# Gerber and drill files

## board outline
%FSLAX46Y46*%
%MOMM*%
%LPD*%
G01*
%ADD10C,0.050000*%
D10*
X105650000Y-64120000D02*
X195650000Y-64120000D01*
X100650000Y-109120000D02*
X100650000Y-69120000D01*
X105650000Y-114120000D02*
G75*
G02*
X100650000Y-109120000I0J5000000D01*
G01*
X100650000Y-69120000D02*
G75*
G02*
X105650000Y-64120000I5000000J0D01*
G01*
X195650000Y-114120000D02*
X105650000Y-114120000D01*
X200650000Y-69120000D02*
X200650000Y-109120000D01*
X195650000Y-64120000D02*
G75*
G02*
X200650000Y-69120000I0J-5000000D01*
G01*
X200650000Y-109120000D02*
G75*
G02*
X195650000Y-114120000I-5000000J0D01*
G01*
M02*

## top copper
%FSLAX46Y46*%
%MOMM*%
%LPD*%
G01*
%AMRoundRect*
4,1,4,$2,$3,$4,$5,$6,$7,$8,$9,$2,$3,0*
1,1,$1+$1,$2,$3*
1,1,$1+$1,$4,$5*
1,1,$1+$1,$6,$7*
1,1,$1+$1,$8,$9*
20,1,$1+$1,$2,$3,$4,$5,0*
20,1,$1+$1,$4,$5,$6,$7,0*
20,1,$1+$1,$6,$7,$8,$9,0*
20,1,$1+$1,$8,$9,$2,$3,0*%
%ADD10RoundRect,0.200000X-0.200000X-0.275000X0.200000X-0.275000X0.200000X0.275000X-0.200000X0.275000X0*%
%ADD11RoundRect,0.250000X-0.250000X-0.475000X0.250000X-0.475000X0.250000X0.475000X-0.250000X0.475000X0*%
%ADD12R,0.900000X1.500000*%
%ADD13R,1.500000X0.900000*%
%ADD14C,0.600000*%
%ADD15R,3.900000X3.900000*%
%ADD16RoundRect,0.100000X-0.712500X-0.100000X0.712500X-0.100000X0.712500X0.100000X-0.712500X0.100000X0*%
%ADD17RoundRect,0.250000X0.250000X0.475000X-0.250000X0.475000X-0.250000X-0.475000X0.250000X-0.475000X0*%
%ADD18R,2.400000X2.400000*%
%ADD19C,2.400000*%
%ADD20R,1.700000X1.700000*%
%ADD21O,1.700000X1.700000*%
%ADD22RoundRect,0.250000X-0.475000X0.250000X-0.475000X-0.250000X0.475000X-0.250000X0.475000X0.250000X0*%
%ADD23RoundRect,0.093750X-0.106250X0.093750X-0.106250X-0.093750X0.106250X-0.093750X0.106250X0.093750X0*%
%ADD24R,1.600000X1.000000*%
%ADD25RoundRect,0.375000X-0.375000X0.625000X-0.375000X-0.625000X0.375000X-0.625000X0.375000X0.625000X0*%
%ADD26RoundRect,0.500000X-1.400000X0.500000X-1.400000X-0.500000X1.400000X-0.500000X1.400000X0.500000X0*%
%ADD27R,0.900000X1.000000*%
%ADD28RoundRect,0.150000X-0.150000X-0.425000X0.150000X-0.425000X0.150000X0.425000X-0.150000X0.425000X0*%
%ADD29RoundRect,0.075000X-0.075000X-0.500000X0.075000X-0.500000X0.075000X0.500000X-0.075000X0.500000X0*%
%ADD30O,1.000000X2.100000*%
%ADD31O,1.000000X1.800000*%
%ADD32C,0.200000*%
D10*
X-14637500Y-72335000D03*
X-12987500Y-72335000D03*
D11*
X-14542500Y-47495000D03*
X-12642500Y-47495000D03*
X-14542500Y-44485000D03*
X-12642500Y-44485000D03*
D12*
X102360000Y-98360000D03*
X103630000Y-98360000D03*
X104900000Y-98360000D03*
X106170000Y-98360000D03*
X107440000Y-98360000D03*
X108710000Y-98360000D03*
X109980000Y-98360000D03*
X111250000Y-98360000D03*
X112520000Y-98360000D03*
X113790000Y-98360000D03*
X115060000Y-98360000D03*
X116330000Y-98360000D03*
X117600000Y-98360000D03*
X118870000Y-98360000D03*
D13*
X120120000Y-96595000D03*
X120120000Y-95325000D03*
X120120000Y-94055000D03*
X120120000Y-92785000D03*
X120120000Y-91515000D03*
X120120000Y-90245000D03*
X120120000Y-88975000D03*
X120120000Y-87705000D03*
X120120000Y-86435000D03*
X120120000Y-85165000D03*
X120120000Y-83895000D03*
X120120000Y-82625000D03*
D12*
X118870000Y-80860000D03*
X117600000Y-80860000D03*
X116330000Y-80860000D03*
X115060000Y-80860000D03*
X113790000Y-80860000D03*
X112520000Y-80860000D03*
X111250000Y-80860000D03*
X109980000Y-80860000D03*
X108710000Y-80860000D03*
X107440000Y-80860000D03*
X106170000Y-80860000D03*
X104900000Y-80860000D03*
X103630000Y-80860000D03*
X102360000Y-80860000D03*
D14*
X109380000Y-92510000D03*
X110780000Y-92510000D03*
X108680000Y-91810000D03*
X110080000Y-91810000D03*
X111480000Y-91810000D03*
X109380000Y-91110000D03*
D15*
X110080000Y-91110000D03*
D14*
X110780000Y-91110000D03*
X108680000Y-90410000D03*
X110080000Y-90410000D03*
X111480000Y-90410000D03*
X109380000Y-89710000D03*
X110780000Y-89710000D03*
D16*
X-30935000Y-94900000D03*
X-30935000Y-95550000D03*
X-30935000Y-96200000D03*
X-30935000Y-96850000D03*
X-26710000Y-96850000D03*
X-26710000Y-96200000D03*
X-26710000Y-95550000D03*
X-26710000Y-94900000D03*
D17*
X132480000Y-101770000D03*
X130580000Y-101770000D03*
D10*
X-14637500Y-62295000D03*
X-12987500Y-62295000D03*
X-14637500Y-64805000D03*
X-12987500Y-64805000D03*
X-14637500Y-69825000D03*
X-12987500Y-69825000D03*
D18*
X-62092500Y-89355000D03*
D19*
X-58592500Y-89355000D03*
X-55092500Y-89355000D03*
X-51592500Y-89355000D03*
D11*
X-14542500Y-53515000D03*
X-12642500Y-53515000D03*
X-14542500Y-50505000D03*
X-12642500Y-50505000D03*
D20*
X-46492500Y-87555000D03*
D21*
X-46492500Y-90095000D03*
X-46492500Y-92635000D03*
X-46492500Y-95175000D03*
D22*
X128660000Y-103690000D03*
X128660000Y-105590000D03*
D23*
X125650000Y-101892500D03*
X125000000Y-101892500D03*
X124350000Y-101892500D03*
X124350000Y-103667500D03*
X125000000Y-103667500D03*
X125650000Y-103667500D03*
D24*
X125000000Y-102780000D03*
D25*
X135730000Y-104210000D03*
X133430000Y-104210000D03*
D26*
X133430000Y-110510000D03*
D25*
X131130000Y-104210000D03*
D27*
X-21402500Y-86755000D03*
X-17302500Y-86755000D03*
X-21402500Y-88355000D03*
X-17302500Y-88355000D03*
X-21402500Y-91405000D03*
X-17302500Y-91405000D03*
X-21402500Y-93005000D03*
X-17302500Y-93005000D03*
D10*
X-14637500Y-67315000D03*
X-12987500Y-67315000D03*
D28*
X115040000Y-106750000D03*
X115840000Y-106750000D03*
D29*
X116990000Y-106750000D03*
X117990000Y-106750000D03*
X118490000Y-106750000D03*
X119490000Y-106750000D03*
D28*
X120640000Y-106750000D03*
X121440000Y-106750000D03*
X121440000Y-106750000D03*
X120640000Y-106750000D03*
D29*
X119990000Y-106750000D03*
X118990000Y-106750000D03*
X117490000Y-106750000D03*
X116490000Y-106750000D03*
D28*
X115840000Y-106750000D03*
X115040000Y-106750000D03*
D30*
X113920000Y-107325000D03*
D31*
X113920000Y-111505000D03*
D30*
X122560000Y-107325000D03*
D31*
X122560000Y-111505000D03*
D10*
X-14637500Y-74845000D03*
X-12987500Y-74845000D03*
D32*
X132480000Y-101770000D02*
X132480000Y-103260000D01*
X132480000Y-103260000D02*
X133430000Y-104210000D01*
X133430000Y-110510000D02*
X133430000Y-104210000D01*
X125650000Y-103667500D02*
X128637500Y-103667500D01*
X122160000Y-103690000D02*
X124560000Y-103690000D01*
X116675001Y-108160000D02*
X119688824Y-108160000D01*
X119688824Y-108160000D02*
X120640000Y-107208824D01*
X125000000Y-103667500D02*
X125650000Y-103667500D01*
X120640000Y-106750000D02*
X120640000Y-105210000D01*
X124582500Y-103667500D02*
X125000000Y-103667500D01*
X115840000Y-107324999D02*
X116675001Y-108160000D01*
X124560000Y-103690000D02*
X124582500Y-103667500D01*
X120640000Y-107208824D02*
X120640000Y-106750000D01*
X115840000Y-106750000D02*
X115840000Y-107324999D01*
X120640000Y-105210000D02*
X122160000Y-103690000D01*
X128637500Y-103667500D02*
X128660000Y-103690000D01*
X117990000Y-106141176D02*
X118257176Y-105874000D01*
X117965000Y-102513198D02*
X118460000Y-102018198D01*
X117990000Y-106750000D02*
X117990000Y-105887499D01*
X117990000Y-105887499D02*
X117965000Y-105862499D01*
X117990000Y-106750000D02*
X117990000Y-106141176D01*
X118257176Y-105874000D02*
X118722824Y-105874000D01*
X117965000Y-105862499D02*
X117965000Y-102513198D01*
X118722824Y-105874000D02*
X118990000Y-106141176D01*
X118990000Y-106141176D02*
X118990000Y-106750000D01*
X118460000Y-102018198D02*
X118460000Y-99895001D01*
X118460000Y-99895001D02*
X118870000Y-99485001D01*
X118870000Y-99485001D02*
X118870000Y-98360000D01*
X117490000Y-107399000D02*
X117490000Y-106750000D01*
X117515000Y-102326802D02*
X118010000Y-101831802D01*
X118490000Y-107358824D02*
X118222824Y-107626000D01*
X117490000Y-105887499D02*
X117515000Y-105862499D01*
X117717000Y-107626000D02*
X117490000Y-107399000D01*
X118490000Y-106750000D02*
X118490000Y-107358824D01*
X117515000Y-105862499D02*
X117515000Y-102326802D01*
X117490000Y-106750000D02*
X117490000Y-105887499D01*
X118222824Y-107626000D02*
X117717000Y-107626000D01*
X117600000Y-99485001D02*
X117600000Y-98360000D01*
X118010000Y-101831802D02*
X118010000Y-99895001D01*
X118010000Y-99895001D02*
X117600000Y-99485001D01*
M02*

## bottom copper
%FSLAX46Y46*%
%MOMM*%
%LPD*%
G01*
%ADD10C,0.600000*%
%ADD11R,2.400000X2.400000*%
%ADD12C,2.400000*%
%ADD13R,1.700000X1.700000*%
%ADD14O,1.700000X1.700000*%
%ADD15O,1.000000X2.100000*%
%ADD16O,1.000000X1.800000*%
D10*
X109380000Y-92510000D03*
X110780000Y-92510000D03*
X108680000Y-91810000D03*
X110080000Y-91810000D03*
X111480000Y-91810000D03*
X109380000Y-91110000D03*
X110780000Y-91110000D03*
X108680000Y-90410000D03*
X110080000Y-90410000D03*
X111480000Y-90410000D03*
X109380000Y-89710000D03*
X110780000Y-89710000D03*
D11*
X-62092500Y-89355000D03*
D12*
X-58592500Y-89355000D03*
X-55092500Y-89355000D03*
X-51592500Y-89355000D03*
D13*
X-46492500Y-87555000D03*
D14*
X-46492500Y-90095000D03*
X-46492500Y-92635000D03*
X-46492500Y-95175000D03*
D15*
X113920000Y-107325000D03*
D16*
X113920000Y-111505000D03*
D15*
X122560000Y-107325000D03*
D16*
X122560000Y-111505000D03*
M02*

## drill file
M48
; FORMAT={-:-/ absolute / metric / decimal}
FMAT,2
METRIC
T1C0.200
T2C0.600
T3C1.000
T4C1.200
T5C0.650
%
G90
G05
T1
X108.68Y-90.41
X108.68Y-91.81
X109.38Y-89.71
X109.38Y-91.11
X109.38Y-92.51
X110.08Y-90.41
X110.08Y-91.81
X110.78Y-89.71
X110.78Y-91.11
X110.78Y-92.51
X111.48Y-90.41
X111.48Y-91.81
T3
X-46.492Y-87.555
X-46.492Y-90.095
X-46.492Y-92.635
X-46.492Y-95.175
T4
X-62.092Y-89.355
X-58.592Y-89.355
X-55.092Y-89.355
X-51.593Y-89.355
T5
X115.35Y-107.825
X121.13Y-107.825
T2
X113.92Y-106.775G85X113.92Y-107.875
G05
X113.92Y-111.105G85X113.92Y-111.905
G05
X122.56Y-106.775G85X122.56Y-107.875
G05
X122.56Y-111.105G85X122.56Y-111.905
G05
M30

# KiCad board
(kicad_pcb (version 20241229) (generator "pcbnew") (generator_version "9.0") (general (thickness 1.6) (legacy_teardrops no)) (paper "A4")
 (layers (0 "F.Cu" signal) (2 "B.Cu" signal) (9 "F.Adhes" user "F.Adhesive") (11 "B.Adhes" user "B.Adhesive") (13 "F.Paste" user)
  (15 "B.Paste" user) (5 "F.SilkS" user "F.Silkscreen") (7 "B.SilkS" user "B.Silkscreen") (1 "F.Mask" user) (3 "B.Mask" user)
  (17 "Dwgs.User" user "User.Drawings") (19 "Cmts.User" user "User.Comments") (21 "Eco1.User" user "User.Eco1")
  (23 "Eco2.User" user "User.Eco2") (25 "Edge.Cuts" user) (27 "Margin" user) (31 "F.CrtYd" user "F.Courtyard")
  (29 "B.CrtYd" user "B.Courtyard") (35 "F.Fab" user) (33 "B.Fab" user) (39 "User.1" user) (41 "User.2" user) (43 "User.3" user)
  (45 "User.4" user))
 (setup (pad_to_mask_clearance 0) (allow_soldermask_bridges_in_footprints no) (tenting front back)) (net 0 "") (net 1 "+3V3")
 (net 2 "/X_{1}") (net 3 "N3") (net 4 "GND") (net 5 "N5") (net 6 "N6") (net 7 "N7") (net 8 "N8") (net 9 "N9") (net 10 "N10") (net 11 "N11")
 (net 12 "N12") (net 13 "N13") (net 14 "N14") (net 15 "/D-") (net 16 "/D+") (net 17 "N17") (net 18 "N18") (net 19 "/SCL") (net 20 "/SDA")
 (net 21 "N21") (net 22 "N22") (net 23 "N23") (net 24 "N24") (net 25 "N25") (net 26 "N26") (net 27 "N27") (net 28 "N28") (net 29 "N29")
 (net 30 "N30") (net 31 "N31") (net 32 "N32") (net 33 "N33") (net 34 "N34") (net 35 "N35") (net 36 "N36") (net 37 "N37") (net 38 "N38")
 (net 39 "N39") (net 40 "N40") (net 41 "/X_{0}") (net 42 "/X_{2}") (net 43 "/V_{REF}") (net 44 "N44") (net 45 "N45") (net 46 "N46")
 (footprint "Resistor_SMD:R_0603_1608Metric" (layer "F.Cu") (at -13.8125 72.335)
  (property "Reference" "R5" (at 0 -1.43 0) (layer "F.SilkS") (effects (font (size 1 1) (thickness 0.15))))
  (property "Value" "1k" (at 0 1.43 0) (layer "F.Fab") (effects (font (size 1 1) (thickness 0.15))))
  (pad "1" smd roundrect (at -0.825 0) (size 0.8 0.95) (layers "F.Cu" "F.Mask" "F.Paste") (roundrect_rratio 0.25) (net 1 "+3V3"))
  (pad "2" smd roundrect (at 0.825 0) (size 0.8 0.95) (layers "F.Cu" "F.Mask" "F.Paste") (roundrect_rratio 0.25) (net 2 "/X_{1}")))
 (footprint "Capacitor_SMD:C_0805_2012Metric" (layer "F.Cu") (at -13.5925 47.495)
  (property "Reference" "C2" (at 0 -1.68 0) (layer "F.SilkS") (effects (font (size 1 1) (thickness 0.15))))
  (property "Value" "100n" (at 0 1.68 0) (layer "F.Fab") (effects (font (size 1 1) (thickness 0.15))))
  (pad "1" smd roundrect (at -0.95 0) (size 1 1.45) (layers "F.Cu" "F.Mask" "F.Paste") (roundrect_rratio 0.25) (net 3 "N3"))
  (pad "2" smd roundrect (at 0.95 0) (size 1 1.45) (layers "F.Cu" "F.Mask" "F.Paste") (roundrect_rratio 0.25) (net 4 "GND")))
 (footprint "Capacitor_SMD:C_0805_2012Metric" (layer "F.Cu") (at -13.5925 44.485)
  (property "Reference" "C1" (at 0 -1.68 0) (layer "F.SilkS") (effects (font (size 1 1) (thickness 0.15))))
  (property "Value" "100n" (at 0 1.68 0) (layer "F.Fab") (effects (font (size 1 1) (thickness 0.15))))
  (pad "1" smd roundrect (at -0.95 0) (size 1 1.45) (layers "F.Cu" "F.Mask" "F.Paste") (roundrect_rratio 0.25) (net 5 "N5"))
  (pad "2" smd roundrect (at 0.95 0) (size 1 1.45) (layers "F.Cu" "F.Mask" "F.Paste") (roundrect_rratio 0.25) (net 4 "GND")))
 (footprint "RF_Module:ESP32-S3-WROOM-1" (layer "F.Cu") (at 107.62 89.61 90)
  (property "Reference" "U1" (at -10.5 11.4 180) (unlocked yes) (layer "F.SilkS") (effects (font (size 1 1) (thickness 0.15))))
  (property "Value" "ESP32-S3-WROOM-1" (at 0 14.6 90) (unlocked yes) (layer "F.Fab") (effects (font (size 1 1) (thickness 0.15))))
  (pad "" smd rect (at -2.9 1.06 90) (size 0.9 0.9) (layers "F.Paste"))
  (pad "" smd rect (at -2.9 2.46) (size 0.9 0.9) (layers "F.Paste"))
  (pad "" smd rect (at -2.9 3.86 90) (size 0.9 0.9) (layers "F.Paste"))
  (pad "" smd rect (at -1.5 1.06) (size 0.9 0.9) (layers "F.Paste"))
  (pad "" smd rect (at -1.5 2.46) (size 0.9 0.9) (layers "F.Paste"))
  (pad "" smd rect (at -1.5 3.86) (size 0.9 0.9) (layers "F.Paste"))
  (pad "" smd rect (at -0.1 1.06) (size 0.9 0.9) (layers "F.Paste"))
  (pad "" smd rect (at -0.1 2.46) (size 0.9 0.9) (layers "F.Paste"))
  (pad "" smd rect (at -0.1 3.86) (size 0.9 0.9) (layers "F.Paste"))
  (pad "1" smd rect (at -8.75 -5.26 90) (size 1.5 0.9) (layers "F.Cu" "F.Mask" "F.Paste") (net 4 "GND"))
  (pad "2" smd rect (at -8.75 -3.99 90) (size 1.5 0.9) (layers "F.Cu" "F.Mask" "F.Paste") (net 1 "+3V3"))
  (pad "3" smd rect (at -8.75 -2.72 90) (size 1.5 0.9) (layers "F.Cu" "F.Mask" "F.Paste") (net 5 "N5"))
  (pad "4" smd rect (at -8.75 -1.45 90) (size 1.5 0.9) (layers "F.Cu" "F.Mask" "F.Paste") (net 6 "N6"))
  (pad "5" smd rect (at -8.75 -0.18 90) (size 1.5 0.9) (layers "F.Cu" "F.Mask" "F.Paste") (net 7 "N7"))
  (pad "6" smd rect (at -8.75 1.09 90) (size 1.5 0.9) (layers "F.Cu" "F.Mask" "F.Paste") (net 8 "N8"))
  (pad "7" smd rect (at -8.75 2.36 90) (size 1.5 0.9) (layers "F.Cu" "F.Mask" "F.Paste") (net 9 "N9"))
  (pad "8" smd rect (at -8.75 3.63 90) (size 1.5 0.9) (layers "F.Cu" "F.Mask" "F.Paste") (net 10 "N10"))
  (pad "9" smd rect (at -8.75 4.9 90) (size 1.5 0.9) (layers "F.Cu" "F.Mask" "F.Paste") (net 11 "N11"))
  (pad "10" smd rect (at -8.75 6.17 90) (size 1.5 0.9) (layers "F.Cu" "F.Mask" "F.Paste") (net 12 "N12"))
  (pad "11" smd rect (at -8.75 7.44 90) (size 1.5 0.9) (layers "F.Cu" "F.Mask" "F.Paste") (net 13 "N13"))
  (pad "12" smd rect (at -8.75 8.71 90) (size 1.5 0.9) (layers "F.Cu" "F.Mask" "F.Paste") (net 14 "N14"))
  (pad "13" smd rect (at -8.75 9.98 90) (size 1.5 0.9) (layers "F.Cu" "F.Mask" "F.Paste") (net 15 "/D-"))
  (pad "14" smd rect (at -8.75 11.25 270) (size 1.5 0.9) (layers "F.Cu" "F.Mask" "F.Paste") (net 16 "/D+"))
  (pad "15" smd rect (at -6.985 12.5) (size 1.5 0.9) (layers "F.Cu" "F.Mask" "F.Paste") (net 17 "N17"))
  (pad "16" smd rect (at -5.715 12.5) (size 1.5 0.9) (layers "F.Cu" "F.Mask" "F.Paste") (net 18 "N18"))
  (pad "17" smd rect (at -4.445 12.5) (size 1.5 0.9) (layers "F.Cu" "F.Mask" "F.Paste") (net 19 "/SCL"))
  (pad "18" smd rect (at -3.175 12.5) (size 1.5 0.9) (layers "F.Cu" "F.Mask" "F.Paste") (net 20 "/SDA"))
  (pad "19" smd rect (at -1.905 12.5) (size 1.5 0.9) (layers "F.Cu" "F.Mask" "F.Paste") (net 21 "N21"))
  (pad "20" smd rect (at -0.635 12.5) (size 1.5 0.9) (layers "F.Cu" "F.Mask" "F.Paste") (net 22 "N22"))
  (pad "21" smd rect (at 0.635 12.5) (size 1.5 0.9) (layers "F.Cu" "F.Mask" "F.Paste") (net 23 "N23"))
  (pad "22" smd rect (at 1.905 12.5) (size 1.5 0.9) (layers "F.Cu" "F.Mask" "F.Paste") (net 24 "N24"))
  (pad "23" smd rect (at 3.175 12.5) (size 1.5 0.9) (layers "F.Cu" "F.Mask" "F.Paste") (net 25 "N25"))
  (pad "24" smd rect (at 4.445 12.5) (size 1.5 0.9) (layers "F.Cu" "F.Mask" "F.Paste") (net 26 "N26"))
  (pad "25" smd rect (at 5.715 12.5) (size 1.5 0.9) (layers "F.Cu" "F.Mask" "F.Paste") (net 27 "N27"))
  (pad "26" smd rect (at 6.985 12.5) (size 1.5 0.9) (layers "F.Cu" "F.Mask" "F.Paste") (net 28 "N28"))
  (pad "27" smd rect (at 8.75 11.25 90) (size 1.5 0.9) (layers "F.Cu" "F.Mask" "F.Paste") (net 3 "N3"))
  (pad "28" smd rect (at 8.75 9.98 90) (size 1.5 0.9) (layers "F.Cu" "F.Mask" "F.Paste") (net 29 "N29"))
  (pad "29" smd rect (at 8.75 8.71 90) (size 1.5 0.9) (layers "F.Cu" "F.Mask" "F.Paste") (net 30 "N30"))
  (pad "30" smd rect (at 8.75 7.44 90) (size 1.5 0.9) (layers "F.Cu" "F.Mask" "F.Paste") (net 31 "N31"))
  (pad "31" smd rect (at 8.75 6.17 90) (size 1.5 0.9) (layers "F.Cu" "F.Mask" "F.Paste") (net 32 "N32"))
  (pad "32" smd rect (at 8.75 4.9 90) (size 1.5 0.9) (layers "F.Cu" "F.Mask" "F.Paste") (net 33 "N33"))
  (pad "33" smd rect (at 8.75 3.63 90) (size 1.5 0.9) (layers "F.Cu" "F.Mask" "F.Paste") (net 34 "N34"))
  (pad "34" smd rect (at 8.75 2.36 90) (size 1.5 0.9) (layers "F.Cu" "F.Mask" "F.Paste") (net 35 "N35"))
  (pad "35" smd rect (at 8.75 1.09 90) (size 1.5 0.9) (layers "F.Cu" "F.Mask" "F.Paste") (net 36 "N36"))
  (pad "36" smd rect (at 8.75 -0.18 90) (size 1.5 0.9) (layers "F.Cu" "F.Mask" "F.Paste") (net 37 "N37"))
  (pad "37" smd rect (at 8.75 -1.45 90) (size 1.5 0.9) (layers "F.Cu" "F.Mask" "F.Paste") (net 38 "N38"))
  (pad "38" smd rect (at 8.75 -2.72 90) (size 1.5 0.9) (layers "F.Cu" "F.Mask" "F.Paste") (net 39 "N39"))
  (pad "39" smd rect (at 8.75 -3.99 90) (size 1.5 0.9) (layers "F.Cu" "F.Mask" "F.Paste") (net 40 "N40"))
  (pad "40" smd rect (at 8.75 -5.26 90) (size 1.5 0.9) (layers "F.Cu" "F.Mask" "F.Paste") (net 4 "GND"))
  (pad "41" thru_hole circle (at -2.9 1.76 180) (size 0.6 0.6) (drill 0.2) (layers "*.Cu" "F.Mask") (remove_unused_layers no) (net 4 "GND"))
  (pad "41" thru_hole circle (at -2.9 3.16 90) (size 0.6 0.6) (drill 0.2) (layers "*.Cu" "F.Mask") (remove_unused_layers no) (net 4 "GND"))
  (pad "41" thru_hole circle (at -2.2 1.06 90) (size 0.6 0.6) (drill 0.2) (layers "*.Cu" "F.Mask") (remove_unused_layers no) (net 4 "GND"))
  (pad "41" thru_hole circle (at -2.2 2.46 90) (size 0.6 0.6) (drill 0.2) (layers "*.Cu" "F.Mask") (remove_unused_layers no) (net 4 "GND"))
  (pad "41" thru_hole circle (at -2.2 3.86 90) (size 0.6 0.6) (drill 0.2) (layers "*.Cu" "F.Mask") (remove_unused_layers no) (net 4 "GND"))
  (pad "41" thru_hole circle (at -1.5 1.76 90) (size 0.6 0.6) (drill 0.2) (layers "*.Cu" "F.Mask") (remove_unused_layers no) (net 4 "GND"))
  (pad "41" smd rect (at -1.5 2.46) (size 3.9 3.9) (layers "F.Cu" "F.Mask") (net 4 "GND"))
  (pad "41" thru_hole circle (at -1.5 3.16 90) (size 0.6 0.6) (drill 0.2) (layers "*.Cu" "F.Mask") (remove_unused_layers no) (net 4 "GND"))
  (pad "41" thru_hole circle (at -0.8 1.06 90) (size 0.6 0.6) (drill 0.2) (layers "*.Cu" "F.Mask") (remove_unused_layers no) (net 4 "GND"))
  (pad "41" thru_hole circle (at -0.8 2.46 90) (size 0.6 0.6) (drill 0.2) (layers "*.Cu" "F.Mask") (remove_unused_layers no) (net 4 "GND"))
  (pad "41" thru_hole circle (at -0.8 3.86 90) (size 0.6 0.6) (drill 0.2) (layers "*.Cu" "F.Mask") (remove_unused_layers no) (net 4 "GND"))
  (pad "41" thru_hole circle (at -0.1 1.76 90) (size 0.6 0.6) (drill 0.2) (layers "*.Cu" "F.Mask") (remove_unused_layers no) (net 4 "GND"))
  (pad "41" thru_hole circle (at -0.1 3.16 90) (size 0.6 0.6) (drill 0.2) (layers "*.Cu" "F.Mask") (remove_unused_layers no) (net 4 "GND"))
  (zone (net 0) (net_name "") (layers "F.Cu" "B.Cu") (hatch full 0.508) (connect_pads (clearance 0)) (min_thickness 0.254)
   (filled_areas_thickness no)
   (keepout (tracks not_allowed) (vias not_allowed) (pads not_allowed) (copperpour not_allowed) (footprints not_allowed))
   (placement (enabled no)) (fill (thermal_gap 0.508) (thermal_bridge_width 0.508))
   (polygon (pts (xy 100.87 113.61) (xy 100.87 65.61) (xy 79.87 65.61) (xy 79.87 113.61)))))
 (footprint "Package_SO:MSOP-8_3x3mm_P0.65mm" (layer "F.Cu") (at -28.8225 95.875)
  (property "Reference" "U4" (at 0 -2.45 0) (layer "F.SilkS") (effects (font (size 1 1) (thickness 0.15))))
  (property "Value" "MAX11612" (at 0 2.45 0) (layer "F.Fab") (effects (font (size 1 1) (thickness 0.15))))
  (pad "1" smd roundrect (at -2.1125 -0.975) (size 1.625 0.4) (layers "F.Cu" "F.Mask" "F.Paste") (roundrect_rratio 0.25) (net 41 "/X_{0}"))
  (pad "2" smd roundrect (at -2.1125 -0.325) (size 1.625 0.4) (layers "F.Cu" "F.Mask" "F.Paste") (roundrect_rratio 0.25) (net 2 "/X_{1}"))
  (pad "3" smd roundrect (at -2.1125 0.325) (size 1.625 0.4) (layers "F.Cu" "F.Mask" "F.Paste") (roundrect_rratio 0.25) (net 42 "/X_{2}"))
  (pad "4" smd roundrect (at -2.1125 0.975) (size 1.625 0.4) (layers "F.Cu" "F.Mask" "F.Paste") (roundrect_rratio 0.25) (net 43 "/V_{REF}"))
  (pad "5" smd roundrect (at 2.1125 0.975) (size 1.625 0.4) (layers "F.Cu" "F.Mask" "F.Paste") (roundrect_rratio 0.25) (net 19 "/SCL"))
  (pad "6" smd roundrect (at 2.1125 0.325) (size 1.625 0.4) (layers "F.Cu" "F.Mask" "F.Paste") (roundrect_rratio 0.25) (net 20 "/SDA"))
  (pad "7" smd roundrect (at 2.1125 -0.325) (size 1.625 0.4) (layers "F.Cu" "F.Mask" "F.Paste") (roundrect_rratio 0.25) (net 4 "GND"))
  (pad "8" smd roundrect (at 2.1125 -0.975) (size 1.625 0.4) (layers "F.Cu" "F.Mask" "F.Paste") (roundrect_rratio 0.25) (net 1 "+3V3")))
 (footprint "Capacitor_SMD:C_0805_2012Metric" (layer "F.Cu") (at 131.53 101.77 180)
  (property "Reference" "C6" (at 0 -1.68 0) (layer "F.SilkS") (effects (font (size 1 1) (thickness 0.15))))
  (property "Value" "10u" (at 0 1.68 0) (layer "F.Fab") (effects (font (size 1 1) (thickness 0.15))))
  (pad "1" smd roundrect (at -0.95 0 180) (size 1 1.45) (layers "F.Cu" "F.Mask" "F.Paste") (roundrect_rratio 0.25) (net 1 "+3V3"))
  (pad "2" smd roundrect (at 0.95 0 180) (size 1 1.45) (layers "F.Cu" "F.Mask" "F.Paste") (roundrect_rratio 0.25) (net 4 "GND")))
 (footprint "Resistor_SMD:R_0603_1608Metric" (layer "F.Cu") (at -13.8125 62.295)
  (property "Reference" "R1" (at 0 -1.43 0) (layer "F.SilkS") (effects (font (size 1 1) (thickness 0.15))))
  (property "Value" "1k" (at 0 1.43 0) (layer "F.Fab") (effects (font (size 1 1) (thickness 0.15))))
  (pad "1" smd roundrect (at -0.825 0) (size 0.8 0.95) (layers "F.Cu" "F.Mask" "F.Paste") (roundrect_rratio 0.25) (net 1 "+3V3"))
  (pad "2" smd roundrect (at 0.825 0) (size 0.8 0.95) (layers "F.Cu" "F.Mask" "F.Paste") (roundrect_rratio 0.25) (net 5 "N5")))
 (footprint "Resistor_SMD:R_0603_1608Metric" (layer "F.Cu") (at -13.8125 64.805)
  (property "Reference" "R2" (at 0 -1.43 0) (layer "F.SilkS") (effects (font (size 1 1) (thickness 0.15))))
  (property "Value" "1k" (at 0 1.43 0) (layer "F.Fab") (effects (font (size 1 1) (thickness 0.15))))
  (pad "1" smd roundrect (at -0.825 0) (size 0.8 0.95) (layers "F.Cu" "F.Mask" "F.Paste") (roundrect_rratio 0.25) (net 1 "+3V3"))
  (pad "2" smd roundrect (at 0.825 0) (size 0.8 0.95) (layers "F.Cu" "F.Mask" "F.Paste") (roundrect_rratio 0.25) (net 3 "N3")))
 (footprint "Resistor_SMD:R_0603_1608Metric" (layer "F.Cu") (at -13.8125 69.825)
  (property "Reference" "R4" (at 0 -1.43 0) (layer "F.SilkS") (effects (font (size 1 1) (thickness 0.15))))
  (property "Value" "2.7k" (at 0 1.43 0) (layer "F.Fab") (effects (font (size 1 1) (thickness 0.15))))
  (pad "1" smd roundrect (at -0.825 0) (size 0.8 0.95) (layers "F.Cu" "F.Mask" "F.Paste") (roundrect_rratio 0.25) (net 1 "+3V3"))
  (pad "2" smd roundrect (at 0.825 0) (size 0.8 0.95) (layers "F.Cu" "F.Mask" "F.Paste") (roundrect_rratio 0.25) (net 20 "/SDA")))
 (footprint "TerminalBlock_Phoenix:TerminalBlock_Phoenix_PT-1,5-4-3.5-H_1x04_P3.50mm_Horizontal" (layer "F.Cu") (at -62.0925 89.355)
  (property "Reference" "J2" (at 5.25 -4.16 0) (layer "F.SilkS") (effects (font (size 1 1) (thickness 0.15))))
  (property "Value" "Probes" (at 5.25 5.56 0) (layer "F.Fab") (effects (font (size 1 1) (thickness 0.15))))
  (pad "1" thru_hole rect (at 0 0) (size 2.4 2.4) (drill 1.2) (layers "*.Cu" "*.Mask") (remove_unused_layers no) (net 41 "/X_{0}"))
  (pad "2" thru_hole circle (at 3.5 0) (size 2.4 2.4) (drill 1.2) (layers "*.Cu" "*.Mask") (remove_unused_layers no) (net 2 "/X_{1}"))
  (pad "3" thru_hole circle (at 7 0) (size 2.4 2.4) (drill 1.2) (layers "*.Cu" "*.Mask") (remove_unused_layers no) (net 42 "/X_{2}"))
  (pad "4" thru_hole circle (at 10.5 0) (size 2.4 2.4) (drill 1.2) (layers "*.Cu" "*.Mask") (remove_unused_layers no) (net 43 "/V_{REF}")))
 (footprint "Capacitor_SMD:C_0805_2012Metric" (layer "F.Cu") (at -13.5925 53.515)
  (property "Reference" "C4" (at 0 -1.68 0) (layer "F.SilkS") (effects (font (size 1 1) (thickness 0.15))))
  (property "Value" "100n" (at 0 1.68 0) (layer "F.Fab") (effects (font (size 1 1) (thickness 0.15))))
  (pad "1" smd roundrect (at -0.95 0) (size 1 1.45) (layers "F.Cu" "F.Mask" "F.Paste") (roundrect_rratio 0.25) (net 1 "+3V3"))
  (pad "2" smd roundrect (at 0.95 0) (size 1 1.45) (layers "F.Cu" "F.Mask" "F.Paste") (roundrect_rratio 0.25) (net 4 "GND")))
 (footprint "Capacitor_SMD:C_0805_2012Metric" (layer "F.Cu") (at -13.5925 50.505)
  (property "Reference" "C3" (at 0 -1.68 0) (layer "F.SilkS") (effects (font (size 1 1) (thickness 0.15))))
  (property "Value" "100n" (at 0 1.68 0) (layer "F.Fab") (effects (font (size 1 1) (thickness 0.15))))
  (pad "1" smd roundrect (at -0.95 0) (size 1 1.45) (layers "F.Cu" "F.Mask" "F.Paste") (roundrect_rratio 0.25) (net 1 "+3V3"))
  (pad "2" smd roundrect (at 0.95 0) (size 1 1.45) (layers "F.Cu" "F.Mask" "F.Paste") (roundrect_rratio 0.25) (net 4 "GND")))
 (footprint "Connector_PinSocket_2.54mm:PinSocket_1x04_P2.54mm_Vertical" (layer "F.Cu") (at -46.4925 87.555)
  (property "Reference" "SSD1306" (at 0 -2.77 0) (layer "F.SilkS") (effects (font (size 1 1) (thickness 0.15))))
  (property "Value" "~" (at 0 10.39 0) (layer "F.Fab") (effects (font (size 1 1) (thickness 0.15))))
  (pad "1" thru_hole rect (at 0 0) (size 1.7 1.7) (drill 1) (layers "*.Cu" "*.Mask") (remove_unused_layers no) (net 4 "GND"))
  (pad "2" thru_hole oval (at 0 2.54) (size 1.7 1.7) (drill 1) (layers "*.Cu" "*.Mask") (remove_unused_layers no) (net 1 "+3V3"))
  (pad "3" thru_hole oval (at 0 5.08) (size 1.7 1.7) (drill 1) (layers "*.Cu" "*.Mask") (remove_unused_layers no) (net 19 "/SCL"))
  (pad "4" thru_hole oval (at 0 7.62) (size 1.7 1.7) (drill 1) (layers "*.Cu" "*.Mask") (remove_unused_layers no) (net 20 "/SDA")))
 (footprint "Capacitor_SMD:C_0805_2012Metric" (layer "F.Cu") (at 128.66 104.64 -90)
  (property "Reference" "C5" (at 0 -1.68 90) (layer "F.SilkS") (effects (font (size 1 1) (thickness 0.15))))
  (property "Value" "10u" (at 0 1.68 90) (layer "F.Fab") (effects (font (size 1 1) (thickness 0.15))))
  (pad "1" smd roundrect (at -0.95 0 270) (size 1 1.45) (layers "F.Cu" "F.Mask" "F.Paste") (roundrect_rratio 0.25) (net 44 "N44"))
  (pad "2" smd roundrect (at 0.95 0 270) (size 1 1.45) (layers "F.Cu" "F.Mask" "F.Paste") (roundrect_rratio 0.25) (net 4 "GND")))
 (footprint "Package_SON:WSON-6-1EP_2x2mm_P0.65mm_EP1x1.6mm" (layer "F.Cu") (at 125 102.78 -90)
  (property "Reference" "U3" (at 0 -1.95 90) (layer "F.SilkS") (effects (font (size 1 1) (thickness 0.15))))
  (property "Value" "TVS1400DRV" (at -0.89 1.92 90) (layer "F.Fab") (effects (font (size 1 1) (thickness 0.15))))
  (pad "" smd roundrect (at 0 -0.4 270) (size 0.81 0.64) (layers "F.Paste") (roundrect_rratio 0.25))
  (pad "" smd roundrect (at 0 0.4 270) (size 0.81 0.64) (layers "F.Paste") (roundrect_rratio 0.25))
  (pad "1" smd roundrect (at -0.8875 -0.65 270) (size 0.375 0.4) (layers "F.Cu" "F.Mask" "F.Paste") (roundrect_rratio 0.25) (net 4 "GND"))
  (pad "2" smd roundrect (at -0.8875 0 270) (size 0.375 0.4) (layers "F.Cu" "F.Mask" "F.Paste") (roundrect_rratio 0.25) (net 4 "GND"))
  (pad "3" smd roundrect (at -0.8875 0.65 270) (size 0.375 0.4) (layers "F.Cu" "F.Mask" "F.Paste") (roundrect_rratio 0.25) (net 4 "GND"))
  (pad "4" smd roundrect (at 0.8875 0.65 270) (size 0.375 0.4) (layers "F.Cu" "F.Mask" "F.Paste") (roundrect_rratio 0.25) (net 44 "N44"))
  (pad "5" smd roundrect (at 0.8875 0 270) (size 0.375 0.4) (layers "F.Cu" "F.Mask" "F.Paste") (roundrect_rratio 0.25) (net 44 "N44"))
  (pad "6" smd roundrect (at 0.8875 -0.65 270) (size 0.375 0.4) (layers "F.Cu" "F.Mask" "F.Paste") (roundrect_rratio 0.25) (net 44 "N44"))
  (pad "7" smd rect (at 0 0 270) (size 1 1.6) (layers "F.Cu" "F.Mask") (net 4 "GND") (zone_connect 2)))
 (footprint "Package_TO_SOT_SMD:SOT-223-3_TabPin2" (layer "F.Cu") (at 133.43 107.36 -90)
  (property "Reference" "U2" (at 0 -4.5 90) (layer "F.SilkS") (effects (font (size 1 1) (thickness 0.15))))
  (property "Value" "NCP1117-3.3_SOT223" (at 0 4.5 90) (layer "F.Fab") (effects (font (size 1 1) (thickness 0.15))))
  (pad "1" smd roundrect (at -3.15 -2.3 270) (size 2 1.5) (layers "F.Cu" "F.Mask" "F.Paste") (roundrect_rratio 0.25) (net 4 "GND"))
  (pad "2" smd roundrect (at -3.15 0 270) (size 2 1.5) (layers "F.Cu" "F.Mask" "F.Paste") (roundrect_rratio 0.25) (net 1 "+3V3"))
  (pad "2" smd roundrect (at 3.15 0 270) (size 2 3.8) (layers "F.Cu" "F.Mask" "F.Paste") (roundrect_rratio 0.25) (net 1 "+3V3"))
  (pad "3" smd roundrect (at -3.15 2.3 270) (size 2 1.5) (layers "F.Cu" "F.Mask" "F.Paste") (roundrect_rratio 0.25) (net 44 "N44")))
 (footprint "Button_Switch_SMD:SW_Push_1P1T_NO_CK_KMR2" (layer "F.Cu") (at -19.3525 87.555)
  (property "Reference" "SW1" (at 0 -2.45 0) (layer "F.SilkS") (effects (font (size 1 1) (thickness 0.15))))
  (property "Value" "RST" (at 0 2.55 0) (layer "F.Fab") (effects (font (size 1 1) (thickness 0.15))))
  (pad "1" smd rect (at -2.05 -0.8) (size 0.9 1) (layers "F.Cu" "F.Mask" "F.Paste") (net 4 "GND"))
  (pad "1" smd rect (at 2.05 -0.8) (size 0.9 1) (layers "F.Cu" "F.Mask" "F.Paste") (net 4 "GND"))
  (pad "2" smd rect (at -2.05 0.8) (size 0.9 1) (layers "F.Cu" "F.Mask" "F.Paste") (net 5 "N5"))
  (pad "2" smd rect (at 2.05 0.8) (size 0.9 1) (layers "F.Cu" "F.Mask" "F.Paste") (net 5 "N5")))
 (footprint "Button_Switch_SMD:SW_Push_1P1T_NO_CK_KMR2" (layer "F.Cu") (at -19.3525 92.205)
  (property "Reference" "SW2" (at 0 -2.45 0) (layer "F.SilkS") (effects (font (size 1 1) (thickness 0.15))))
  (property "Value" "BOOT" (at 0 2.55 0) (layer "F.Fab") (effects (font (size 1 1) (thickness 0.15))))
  (pad "1" smd rect (at -2.05 -0.8) (size 0.9 1) (layers "F.Cu" "F.Mask" "F.Paste") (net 4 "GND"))
  (pad "1" smd rect (at 2.05 -0.8) (size 0.9 1) (layers "F.Cu" "F.Mask" "F.Paste") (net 4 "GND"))
  (pad "2" smd rect (at -2.05 0.8) (size 0.9 1) (layers "F.Cu" "F.Mask" "F.Paste") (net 3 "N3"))
  (pad "2" smd rect (at 2.05 0.8) (size 0.9 1) (layers "F.Cu" "F.Mask" "F.Paste") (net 3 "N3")))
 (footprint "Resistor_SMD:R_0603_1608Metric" (layer "F.Cu") (at -13.8125 67.315)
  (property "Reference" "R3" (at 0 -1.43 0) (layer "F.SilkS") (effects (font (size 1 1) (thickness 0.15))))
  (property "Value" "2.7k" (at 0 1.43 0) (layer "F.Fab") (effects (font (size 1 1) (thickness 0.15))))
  (pad "1" smd roundrect (at -0.825 0) (size 0.8 0.95) (layers "F.Cu" "F.Mask" "F.Paste") (roundrect_rratio 0.25) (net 1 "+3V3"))
  (pad "2" smd roundrect (at 0.825 0) (size 0.8 0.95) (layers "F.Cu" "F.Mask" "F.Paste") (roundrect_rratio 0.25) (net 19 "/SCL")))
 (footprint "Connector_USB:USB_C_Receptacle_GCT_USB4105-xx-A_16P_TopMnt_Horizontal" (layer "F.Cu") (at 118.24 110.43)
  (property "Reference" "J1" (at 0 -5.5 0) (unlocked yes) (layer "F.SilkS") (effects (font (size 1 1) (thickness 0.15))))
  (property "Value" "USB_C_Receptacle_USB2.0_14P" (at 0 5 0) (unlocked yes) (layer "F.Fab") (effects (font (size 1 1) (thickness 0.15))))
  (pad "" np_thru_hole circle (at -2.89 -2.605) (size 0.65 0.65) (drill 0.65) (layers "*.Cu" "*.Mask"))
  (pad "" np_thru_hole circle (at 2.89 -2.605) (size 0.65 0.65) (drill 0.65) (layers "*.Cu" "*.Mask"))
  (pad "A1" smd roundrect (at -3.2 -3.68) (size 0.6 1.15) (layers "F.Cu" "F.Mask" "F.Paste") (roundrect_rratio 0.25) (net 4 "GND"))
  (pad "A4" smd roundrect (at -2.4 -3.68) (size 0.6 1.15) (layers "F.Cu" "F.Mask" "F.Paste") (roundrect_rratio 0.25) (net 44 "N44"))
  (pad "A5" smd roundrect (at -1.25 -3.68) (size 0.3 1.15) (layers "F.Cu" "F.Mask" "F.Paste") (roundrect_rratio 0.25) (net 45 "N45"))
  (pad "A6" smd roundrect (at -0.25 -3.68) (size 0.3 1.15) (layers "F.Cu" "F.Mask" "F.Paste") (roundrect_rratio 0.25) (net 16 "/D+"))
  (pad "A7" smd roundrect (at 0.25 -3.68) (size 0.3 1.15) (layers "F.Cu" "F.Mask" "F.Paste") (roundrect_rratio 0.25) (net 15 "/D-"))
  (pad "A8" smd roundrect (at 1.25 -3.68) (size 0.3 1.15) (layers "F.Cu" "F.Mask" "F.Paste") (roundrect_rratio 0.25))
  (pad "A9" smd roundrect (at 2.4 -3.68) (size 0.6 1.15) (layers "F.Cu" "F.Mask" "F.Paste") (roundrect_rratio 0.25) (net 44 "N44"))
  (pad "A12" smd roundrect (at 3.2 -3.68) (size 0.6 1.15) (layers "F.Cu" "F.Mask" "F.Paste") (roundrect_rratio 0.25) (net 4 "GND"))
  (pad "B1" smd roundrect (at 3.2 -3.68) (size 0.6 1.15) (layers "F.Cu" "F.Mask" "F.Paste") (roundrect_rratio 0.25) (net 4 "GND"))
  (pad "B4" smd roundrect (at 2.4 -3.68) (size 0.6 1.15) (layers "F.Cu" "F.Mask" "F.Paste") (roundrect_rratio 0.25) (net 44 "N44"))
  (pad "B5" smd roundrect (at 1.75 -3.68) (size 0.3 1.15) (layers "F.Cu" "F.Mask" "F.Paste") (roundrect_rratio 0.25) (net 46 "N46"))
  (pad "B6" smd roundrect (at 0.75 -3.68) (size 0.3 1.15) (layers "F.Cu" "F.Mask" "F.Paste") (roundrect_rratio 0.25) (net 16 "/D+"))
  (pad "B7" smd roundrect (at -0.75 -3.68) (size 0.3 1.15) (layers "F.Cu" "F.Mask" "F.Paste") (roundrect_rratio 0.25) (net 15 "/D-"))
  (pad "B8" smd roundrect (at -1.75 -3.68) (size 0.3 1.15) (layers "F.Cu" "F.Mask" "F.Paste") (roundrect_rratio 0.25))
  (pad "B9" smd roundrect (at -2.4 -3.68) (size 0.6 1.15) (layers "F.Cu" "F.Mask" "F.Paste") (roundrect_rratio 0.25) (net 44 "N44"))
  (pad "B12" smd roundrect (at -3.2 -3.68) (size 0.6 1.15) (layers "F.Cu" "F.Mask" "F.Paste") (roundrect_rratio 0.25) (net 4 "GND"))
  (pad "S1" thru_hole oval (at -4.32 -3.105) (size 1 2.1) (drill oval 0.6 1.7) (layers "*.Cu" "*.Mask" "F.Paste") (remove_unused_layers no)
   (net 4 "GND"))
  (pad "S1" thru_hole oval (at -4.32 1.075) (size 1 1.8) (drill oval 0.6 1.4) (layers "*.Cu" "*.Mask" "F.Paste") (remove_unused_layers no)
   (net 4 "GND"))
  (pad "S1" thru_hole oval (at 4.32 -3.105) (size 1 2.1) (drill oval 0.6 1.7) (layers "*.Cu" "*.Mask" "F.Paste") (remove_unused_layers no)
   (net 4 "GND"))
  (pad "S1" thru_hole oval (at 4.32 1.075) (size 1 1.8) (drill oval 0.6 1.4) (layers "*.Cu" "*.Mask" "F.Paste") (remove_unused_layers no)
   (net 4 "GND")))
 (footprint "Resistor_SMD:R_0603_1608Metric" (layer "F.Cu") (at -13.8125 74.845)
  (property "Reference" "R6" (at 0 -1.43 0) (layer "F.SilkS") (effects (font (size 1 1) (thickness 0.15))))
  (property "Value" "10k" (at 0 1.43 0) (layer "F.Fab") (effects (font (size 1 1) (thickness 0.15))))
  (pad "1" smd roundrect (at -0.825 0) (size 0.8 0.95) (layers "F.Cu" "F.Mask" "F.Paste") (roundrect_rratio 0.25) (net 1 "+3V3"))
  (pad "2" smd roundrect (at 0.825 0) (size 0.8 0.95) (layers "F.Cu" "F.Mask" "F.Paste") (roundrect_rratio 0.25) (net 42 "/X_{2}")))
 (gr_line (start 105.65 64.12) (end 195.65 64.12) (stroke (width 0.05) (type default)) (locked yes) (layer "Edge.Cuts"))
 (gr_line (start 100.65 109.12) (end 100.65 69.12) (stroke (width 0.05) (type default)) (locked yes) (layer "Edge.Cuts"))
 (gr_arc (start 105.65 114.12) (mid 102.114466 112.655534) (end 100.65 109.12) (stroke (width 0.05) (type default)) (locked yes)
  (layer "Edge.Cuts"))
 (gr_arc (start 100.65 69.12) (mid 102.114466 65.584466) (end 105.65 64.12) (stroke (width 0.05) (type default)) (locked yes)
  (layer "Edge.Cuts"))
 (gr_line (start 195.65 114.12) (end 105.65 114.12) (stroke (width 0.05) (type default)) (locked yes) (layer "Edge.Cuts"))
 (gr_line (start 200.65 69.12) (end 200.65 109.12) (stroke (width 0.05) (type default)) (locked yes) (layer "Edge.Cuts"))
 (gr_arc (start 195.65 64.12) (mid 199.185534 65.584466) (end 200.65 69.12) (stroke (width 0.05) (type default)) (locked yes)
  (layer "Edge.Cuts"))
 (gr_arc (start 200.65 109.12) (mid 199.185534 112.655534) (end 195.65 114.12) (stroke (width 0.05) (type default)) (locked yes)
  (layer "Edge.Cuts"))
 (segment (start 132.48 101.77) (end 132.48 103.26) (width 0.2) (layer "F.Cu") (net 1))
 (segment (start 132.48 103.26) (end 133.43 104.21) (width 0.2) (layer "F.Cu") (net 1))
 (segment (start 133.43 110.51) (end 133.43 104.21) (width 0.2) (layer "F.Cu") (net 1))
 (segment (start 125.65 103.6675) (end 128.6375 103.6675) (width 0.2) (layer "F.Cu") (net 44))
 (segment (start 122.16 103.69) (end 124.56 103.69) (width 0.2) (layer "F.Cu") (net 44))
 (segment (start 116.675001 108.16) (end 119.688824 108.16) (width 0.2) (layer "F.Cu") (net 44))
 (segment (start 119.688824 108.16) (end 120.64 107.208824) (width 0.2) (layer "F.Cu") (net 44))
 (segment (start 125 103.6675) (end 125.65 103.6675) (width 0.2) (layer "F.Cu") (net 44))
 (segment (start 120.64 106.75) (end 120.64 105.21) (width 0.2) (layer "F.Cu") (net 44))
 (segment (start 124.5825 103.6675) (end 125 103.6675) (width 0.2) (layer "F.Cu") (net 44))
 (segment (start 115.84 107.324999) (end 116.675001 108.16) (width 0.2) (layer "F.Cu") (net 44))
 (segment (start 124.56 103.69) (end 124.5825 103.6675) (width 0.2) (layer "F.Cu") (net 44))
 (segment (start 120.64 107.208824) (end 120.64 106.75) (width 0.2) (layer "F.Cu") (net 44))
 (segment (start 115.84 106.75) (end 115.84 107.324999) (width 0.2) (layer "F.Cu") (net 44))
 (segment (start 120.64 105.21) (end 122.16 103.69) (width 0.2) (layer "F.Cu") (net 44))
 (segment (start 128.6375 103.6675) (end 128.66 103.69) (width 0.2) (layer "F.Cu") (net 44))
 (segment (start 117.99 106.141176) (end 118.257176 105.874) (width 0.2) (layer "F.Cu") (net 16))
 (segment (start 117.965 102.513198) (end 118.46 102.018198) (width 0.2) (layer "F.Cu") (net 16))
 (segment (start 117.99 106.75) (end 117.99 105.887499) (width 0.2) (layer "F.Cu") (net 16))
 (segment (start 117.99 105.887499) (end 117.965 105.862499) (width 0.2) (layer "F.Cu") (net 16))
 (segment (start 117.99 106.75) (end 117.99 106.141176) (width 0.2) (layer "F.Cu") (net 16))
 (segment (start 118.257176 105.874) (end 118.722824 105.874) (width 0.2) (layer "F.Cu") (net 16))
 (segment (start 117.965 105.862499) (end 117.965 102.513198) (width 0.2) (layer "F.Cu") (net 16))
 (segment (start 118.722824 105.874) (end 118.99 106.141176) (width 0.2) (layer "F.Cu") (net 16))
 (segment (start 118.99 106.141176) (end 118.99 106.75) (width 0.2) (layer "F.Cu") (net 16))
 (segment (start 118.46 102.018198) (end 118.46 99.895001) (width 0.2) (layer "F.Cu") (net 16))
 (segment (start 118.46 99.895001) (end 118.87 99.485001) (width 0.2) (layer "F.Cu") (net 16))
 (segment (start 118.87 99.485001) (end 118.87 98.36) (width 0.2) (layer "F.Cu") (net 16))
 (segment (start 117.49 107.399) (end 117.49 106.75) (width 0.2) (layer "F.Cu") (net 15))
 (segment (start 117.515 102.326802) (end 118.01 101.831802) (width 0.2) (layer "F.Cu") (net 15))
 (segment (start 118.49 107.358824) (end 118.222824 107.626) (width 0.2) (layer "F.Cu") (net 15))
 (segment (start 117.49 105.887499) (end 117.515 105.862499) (width 0.2) (layer "F.Cu") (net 15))
 (segment (start 117.717 107.626) (end 117.49 107.399) (width 0.2) (layer "F.Cu") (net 15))
 (segment (start 118.49 106.75) (end 118.49 107.358824) (width 0.2) (layer "F.Cu") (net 15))
 (segment (start 117.515 105.862499) (end 117.515 102.326802) (width 0.2) (layer "F.Cu") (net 15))
 (segment (start 117.49 106.75) (end 117.49 105.887499) (width 0.2) (layer "F.Cu") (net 15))
 (segment (start 118.222824 107.626) (end 117.717 107.626) (width 0.2) (layer "F.Cu") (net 15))
 (segment (start 117.6 99.485001) (end 117.6 98.36) (width 0.2) (layer "F.Cu") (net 15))
 (segment (start 118.01 101.831802) (end 118.01 99.895001) (width 0.2) (layer "F.Cu") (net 15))
 (segment (start 118.01 99.895001) (end 117.6 99.485001) (width 0.2) (layer "F.Cu") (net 15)))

